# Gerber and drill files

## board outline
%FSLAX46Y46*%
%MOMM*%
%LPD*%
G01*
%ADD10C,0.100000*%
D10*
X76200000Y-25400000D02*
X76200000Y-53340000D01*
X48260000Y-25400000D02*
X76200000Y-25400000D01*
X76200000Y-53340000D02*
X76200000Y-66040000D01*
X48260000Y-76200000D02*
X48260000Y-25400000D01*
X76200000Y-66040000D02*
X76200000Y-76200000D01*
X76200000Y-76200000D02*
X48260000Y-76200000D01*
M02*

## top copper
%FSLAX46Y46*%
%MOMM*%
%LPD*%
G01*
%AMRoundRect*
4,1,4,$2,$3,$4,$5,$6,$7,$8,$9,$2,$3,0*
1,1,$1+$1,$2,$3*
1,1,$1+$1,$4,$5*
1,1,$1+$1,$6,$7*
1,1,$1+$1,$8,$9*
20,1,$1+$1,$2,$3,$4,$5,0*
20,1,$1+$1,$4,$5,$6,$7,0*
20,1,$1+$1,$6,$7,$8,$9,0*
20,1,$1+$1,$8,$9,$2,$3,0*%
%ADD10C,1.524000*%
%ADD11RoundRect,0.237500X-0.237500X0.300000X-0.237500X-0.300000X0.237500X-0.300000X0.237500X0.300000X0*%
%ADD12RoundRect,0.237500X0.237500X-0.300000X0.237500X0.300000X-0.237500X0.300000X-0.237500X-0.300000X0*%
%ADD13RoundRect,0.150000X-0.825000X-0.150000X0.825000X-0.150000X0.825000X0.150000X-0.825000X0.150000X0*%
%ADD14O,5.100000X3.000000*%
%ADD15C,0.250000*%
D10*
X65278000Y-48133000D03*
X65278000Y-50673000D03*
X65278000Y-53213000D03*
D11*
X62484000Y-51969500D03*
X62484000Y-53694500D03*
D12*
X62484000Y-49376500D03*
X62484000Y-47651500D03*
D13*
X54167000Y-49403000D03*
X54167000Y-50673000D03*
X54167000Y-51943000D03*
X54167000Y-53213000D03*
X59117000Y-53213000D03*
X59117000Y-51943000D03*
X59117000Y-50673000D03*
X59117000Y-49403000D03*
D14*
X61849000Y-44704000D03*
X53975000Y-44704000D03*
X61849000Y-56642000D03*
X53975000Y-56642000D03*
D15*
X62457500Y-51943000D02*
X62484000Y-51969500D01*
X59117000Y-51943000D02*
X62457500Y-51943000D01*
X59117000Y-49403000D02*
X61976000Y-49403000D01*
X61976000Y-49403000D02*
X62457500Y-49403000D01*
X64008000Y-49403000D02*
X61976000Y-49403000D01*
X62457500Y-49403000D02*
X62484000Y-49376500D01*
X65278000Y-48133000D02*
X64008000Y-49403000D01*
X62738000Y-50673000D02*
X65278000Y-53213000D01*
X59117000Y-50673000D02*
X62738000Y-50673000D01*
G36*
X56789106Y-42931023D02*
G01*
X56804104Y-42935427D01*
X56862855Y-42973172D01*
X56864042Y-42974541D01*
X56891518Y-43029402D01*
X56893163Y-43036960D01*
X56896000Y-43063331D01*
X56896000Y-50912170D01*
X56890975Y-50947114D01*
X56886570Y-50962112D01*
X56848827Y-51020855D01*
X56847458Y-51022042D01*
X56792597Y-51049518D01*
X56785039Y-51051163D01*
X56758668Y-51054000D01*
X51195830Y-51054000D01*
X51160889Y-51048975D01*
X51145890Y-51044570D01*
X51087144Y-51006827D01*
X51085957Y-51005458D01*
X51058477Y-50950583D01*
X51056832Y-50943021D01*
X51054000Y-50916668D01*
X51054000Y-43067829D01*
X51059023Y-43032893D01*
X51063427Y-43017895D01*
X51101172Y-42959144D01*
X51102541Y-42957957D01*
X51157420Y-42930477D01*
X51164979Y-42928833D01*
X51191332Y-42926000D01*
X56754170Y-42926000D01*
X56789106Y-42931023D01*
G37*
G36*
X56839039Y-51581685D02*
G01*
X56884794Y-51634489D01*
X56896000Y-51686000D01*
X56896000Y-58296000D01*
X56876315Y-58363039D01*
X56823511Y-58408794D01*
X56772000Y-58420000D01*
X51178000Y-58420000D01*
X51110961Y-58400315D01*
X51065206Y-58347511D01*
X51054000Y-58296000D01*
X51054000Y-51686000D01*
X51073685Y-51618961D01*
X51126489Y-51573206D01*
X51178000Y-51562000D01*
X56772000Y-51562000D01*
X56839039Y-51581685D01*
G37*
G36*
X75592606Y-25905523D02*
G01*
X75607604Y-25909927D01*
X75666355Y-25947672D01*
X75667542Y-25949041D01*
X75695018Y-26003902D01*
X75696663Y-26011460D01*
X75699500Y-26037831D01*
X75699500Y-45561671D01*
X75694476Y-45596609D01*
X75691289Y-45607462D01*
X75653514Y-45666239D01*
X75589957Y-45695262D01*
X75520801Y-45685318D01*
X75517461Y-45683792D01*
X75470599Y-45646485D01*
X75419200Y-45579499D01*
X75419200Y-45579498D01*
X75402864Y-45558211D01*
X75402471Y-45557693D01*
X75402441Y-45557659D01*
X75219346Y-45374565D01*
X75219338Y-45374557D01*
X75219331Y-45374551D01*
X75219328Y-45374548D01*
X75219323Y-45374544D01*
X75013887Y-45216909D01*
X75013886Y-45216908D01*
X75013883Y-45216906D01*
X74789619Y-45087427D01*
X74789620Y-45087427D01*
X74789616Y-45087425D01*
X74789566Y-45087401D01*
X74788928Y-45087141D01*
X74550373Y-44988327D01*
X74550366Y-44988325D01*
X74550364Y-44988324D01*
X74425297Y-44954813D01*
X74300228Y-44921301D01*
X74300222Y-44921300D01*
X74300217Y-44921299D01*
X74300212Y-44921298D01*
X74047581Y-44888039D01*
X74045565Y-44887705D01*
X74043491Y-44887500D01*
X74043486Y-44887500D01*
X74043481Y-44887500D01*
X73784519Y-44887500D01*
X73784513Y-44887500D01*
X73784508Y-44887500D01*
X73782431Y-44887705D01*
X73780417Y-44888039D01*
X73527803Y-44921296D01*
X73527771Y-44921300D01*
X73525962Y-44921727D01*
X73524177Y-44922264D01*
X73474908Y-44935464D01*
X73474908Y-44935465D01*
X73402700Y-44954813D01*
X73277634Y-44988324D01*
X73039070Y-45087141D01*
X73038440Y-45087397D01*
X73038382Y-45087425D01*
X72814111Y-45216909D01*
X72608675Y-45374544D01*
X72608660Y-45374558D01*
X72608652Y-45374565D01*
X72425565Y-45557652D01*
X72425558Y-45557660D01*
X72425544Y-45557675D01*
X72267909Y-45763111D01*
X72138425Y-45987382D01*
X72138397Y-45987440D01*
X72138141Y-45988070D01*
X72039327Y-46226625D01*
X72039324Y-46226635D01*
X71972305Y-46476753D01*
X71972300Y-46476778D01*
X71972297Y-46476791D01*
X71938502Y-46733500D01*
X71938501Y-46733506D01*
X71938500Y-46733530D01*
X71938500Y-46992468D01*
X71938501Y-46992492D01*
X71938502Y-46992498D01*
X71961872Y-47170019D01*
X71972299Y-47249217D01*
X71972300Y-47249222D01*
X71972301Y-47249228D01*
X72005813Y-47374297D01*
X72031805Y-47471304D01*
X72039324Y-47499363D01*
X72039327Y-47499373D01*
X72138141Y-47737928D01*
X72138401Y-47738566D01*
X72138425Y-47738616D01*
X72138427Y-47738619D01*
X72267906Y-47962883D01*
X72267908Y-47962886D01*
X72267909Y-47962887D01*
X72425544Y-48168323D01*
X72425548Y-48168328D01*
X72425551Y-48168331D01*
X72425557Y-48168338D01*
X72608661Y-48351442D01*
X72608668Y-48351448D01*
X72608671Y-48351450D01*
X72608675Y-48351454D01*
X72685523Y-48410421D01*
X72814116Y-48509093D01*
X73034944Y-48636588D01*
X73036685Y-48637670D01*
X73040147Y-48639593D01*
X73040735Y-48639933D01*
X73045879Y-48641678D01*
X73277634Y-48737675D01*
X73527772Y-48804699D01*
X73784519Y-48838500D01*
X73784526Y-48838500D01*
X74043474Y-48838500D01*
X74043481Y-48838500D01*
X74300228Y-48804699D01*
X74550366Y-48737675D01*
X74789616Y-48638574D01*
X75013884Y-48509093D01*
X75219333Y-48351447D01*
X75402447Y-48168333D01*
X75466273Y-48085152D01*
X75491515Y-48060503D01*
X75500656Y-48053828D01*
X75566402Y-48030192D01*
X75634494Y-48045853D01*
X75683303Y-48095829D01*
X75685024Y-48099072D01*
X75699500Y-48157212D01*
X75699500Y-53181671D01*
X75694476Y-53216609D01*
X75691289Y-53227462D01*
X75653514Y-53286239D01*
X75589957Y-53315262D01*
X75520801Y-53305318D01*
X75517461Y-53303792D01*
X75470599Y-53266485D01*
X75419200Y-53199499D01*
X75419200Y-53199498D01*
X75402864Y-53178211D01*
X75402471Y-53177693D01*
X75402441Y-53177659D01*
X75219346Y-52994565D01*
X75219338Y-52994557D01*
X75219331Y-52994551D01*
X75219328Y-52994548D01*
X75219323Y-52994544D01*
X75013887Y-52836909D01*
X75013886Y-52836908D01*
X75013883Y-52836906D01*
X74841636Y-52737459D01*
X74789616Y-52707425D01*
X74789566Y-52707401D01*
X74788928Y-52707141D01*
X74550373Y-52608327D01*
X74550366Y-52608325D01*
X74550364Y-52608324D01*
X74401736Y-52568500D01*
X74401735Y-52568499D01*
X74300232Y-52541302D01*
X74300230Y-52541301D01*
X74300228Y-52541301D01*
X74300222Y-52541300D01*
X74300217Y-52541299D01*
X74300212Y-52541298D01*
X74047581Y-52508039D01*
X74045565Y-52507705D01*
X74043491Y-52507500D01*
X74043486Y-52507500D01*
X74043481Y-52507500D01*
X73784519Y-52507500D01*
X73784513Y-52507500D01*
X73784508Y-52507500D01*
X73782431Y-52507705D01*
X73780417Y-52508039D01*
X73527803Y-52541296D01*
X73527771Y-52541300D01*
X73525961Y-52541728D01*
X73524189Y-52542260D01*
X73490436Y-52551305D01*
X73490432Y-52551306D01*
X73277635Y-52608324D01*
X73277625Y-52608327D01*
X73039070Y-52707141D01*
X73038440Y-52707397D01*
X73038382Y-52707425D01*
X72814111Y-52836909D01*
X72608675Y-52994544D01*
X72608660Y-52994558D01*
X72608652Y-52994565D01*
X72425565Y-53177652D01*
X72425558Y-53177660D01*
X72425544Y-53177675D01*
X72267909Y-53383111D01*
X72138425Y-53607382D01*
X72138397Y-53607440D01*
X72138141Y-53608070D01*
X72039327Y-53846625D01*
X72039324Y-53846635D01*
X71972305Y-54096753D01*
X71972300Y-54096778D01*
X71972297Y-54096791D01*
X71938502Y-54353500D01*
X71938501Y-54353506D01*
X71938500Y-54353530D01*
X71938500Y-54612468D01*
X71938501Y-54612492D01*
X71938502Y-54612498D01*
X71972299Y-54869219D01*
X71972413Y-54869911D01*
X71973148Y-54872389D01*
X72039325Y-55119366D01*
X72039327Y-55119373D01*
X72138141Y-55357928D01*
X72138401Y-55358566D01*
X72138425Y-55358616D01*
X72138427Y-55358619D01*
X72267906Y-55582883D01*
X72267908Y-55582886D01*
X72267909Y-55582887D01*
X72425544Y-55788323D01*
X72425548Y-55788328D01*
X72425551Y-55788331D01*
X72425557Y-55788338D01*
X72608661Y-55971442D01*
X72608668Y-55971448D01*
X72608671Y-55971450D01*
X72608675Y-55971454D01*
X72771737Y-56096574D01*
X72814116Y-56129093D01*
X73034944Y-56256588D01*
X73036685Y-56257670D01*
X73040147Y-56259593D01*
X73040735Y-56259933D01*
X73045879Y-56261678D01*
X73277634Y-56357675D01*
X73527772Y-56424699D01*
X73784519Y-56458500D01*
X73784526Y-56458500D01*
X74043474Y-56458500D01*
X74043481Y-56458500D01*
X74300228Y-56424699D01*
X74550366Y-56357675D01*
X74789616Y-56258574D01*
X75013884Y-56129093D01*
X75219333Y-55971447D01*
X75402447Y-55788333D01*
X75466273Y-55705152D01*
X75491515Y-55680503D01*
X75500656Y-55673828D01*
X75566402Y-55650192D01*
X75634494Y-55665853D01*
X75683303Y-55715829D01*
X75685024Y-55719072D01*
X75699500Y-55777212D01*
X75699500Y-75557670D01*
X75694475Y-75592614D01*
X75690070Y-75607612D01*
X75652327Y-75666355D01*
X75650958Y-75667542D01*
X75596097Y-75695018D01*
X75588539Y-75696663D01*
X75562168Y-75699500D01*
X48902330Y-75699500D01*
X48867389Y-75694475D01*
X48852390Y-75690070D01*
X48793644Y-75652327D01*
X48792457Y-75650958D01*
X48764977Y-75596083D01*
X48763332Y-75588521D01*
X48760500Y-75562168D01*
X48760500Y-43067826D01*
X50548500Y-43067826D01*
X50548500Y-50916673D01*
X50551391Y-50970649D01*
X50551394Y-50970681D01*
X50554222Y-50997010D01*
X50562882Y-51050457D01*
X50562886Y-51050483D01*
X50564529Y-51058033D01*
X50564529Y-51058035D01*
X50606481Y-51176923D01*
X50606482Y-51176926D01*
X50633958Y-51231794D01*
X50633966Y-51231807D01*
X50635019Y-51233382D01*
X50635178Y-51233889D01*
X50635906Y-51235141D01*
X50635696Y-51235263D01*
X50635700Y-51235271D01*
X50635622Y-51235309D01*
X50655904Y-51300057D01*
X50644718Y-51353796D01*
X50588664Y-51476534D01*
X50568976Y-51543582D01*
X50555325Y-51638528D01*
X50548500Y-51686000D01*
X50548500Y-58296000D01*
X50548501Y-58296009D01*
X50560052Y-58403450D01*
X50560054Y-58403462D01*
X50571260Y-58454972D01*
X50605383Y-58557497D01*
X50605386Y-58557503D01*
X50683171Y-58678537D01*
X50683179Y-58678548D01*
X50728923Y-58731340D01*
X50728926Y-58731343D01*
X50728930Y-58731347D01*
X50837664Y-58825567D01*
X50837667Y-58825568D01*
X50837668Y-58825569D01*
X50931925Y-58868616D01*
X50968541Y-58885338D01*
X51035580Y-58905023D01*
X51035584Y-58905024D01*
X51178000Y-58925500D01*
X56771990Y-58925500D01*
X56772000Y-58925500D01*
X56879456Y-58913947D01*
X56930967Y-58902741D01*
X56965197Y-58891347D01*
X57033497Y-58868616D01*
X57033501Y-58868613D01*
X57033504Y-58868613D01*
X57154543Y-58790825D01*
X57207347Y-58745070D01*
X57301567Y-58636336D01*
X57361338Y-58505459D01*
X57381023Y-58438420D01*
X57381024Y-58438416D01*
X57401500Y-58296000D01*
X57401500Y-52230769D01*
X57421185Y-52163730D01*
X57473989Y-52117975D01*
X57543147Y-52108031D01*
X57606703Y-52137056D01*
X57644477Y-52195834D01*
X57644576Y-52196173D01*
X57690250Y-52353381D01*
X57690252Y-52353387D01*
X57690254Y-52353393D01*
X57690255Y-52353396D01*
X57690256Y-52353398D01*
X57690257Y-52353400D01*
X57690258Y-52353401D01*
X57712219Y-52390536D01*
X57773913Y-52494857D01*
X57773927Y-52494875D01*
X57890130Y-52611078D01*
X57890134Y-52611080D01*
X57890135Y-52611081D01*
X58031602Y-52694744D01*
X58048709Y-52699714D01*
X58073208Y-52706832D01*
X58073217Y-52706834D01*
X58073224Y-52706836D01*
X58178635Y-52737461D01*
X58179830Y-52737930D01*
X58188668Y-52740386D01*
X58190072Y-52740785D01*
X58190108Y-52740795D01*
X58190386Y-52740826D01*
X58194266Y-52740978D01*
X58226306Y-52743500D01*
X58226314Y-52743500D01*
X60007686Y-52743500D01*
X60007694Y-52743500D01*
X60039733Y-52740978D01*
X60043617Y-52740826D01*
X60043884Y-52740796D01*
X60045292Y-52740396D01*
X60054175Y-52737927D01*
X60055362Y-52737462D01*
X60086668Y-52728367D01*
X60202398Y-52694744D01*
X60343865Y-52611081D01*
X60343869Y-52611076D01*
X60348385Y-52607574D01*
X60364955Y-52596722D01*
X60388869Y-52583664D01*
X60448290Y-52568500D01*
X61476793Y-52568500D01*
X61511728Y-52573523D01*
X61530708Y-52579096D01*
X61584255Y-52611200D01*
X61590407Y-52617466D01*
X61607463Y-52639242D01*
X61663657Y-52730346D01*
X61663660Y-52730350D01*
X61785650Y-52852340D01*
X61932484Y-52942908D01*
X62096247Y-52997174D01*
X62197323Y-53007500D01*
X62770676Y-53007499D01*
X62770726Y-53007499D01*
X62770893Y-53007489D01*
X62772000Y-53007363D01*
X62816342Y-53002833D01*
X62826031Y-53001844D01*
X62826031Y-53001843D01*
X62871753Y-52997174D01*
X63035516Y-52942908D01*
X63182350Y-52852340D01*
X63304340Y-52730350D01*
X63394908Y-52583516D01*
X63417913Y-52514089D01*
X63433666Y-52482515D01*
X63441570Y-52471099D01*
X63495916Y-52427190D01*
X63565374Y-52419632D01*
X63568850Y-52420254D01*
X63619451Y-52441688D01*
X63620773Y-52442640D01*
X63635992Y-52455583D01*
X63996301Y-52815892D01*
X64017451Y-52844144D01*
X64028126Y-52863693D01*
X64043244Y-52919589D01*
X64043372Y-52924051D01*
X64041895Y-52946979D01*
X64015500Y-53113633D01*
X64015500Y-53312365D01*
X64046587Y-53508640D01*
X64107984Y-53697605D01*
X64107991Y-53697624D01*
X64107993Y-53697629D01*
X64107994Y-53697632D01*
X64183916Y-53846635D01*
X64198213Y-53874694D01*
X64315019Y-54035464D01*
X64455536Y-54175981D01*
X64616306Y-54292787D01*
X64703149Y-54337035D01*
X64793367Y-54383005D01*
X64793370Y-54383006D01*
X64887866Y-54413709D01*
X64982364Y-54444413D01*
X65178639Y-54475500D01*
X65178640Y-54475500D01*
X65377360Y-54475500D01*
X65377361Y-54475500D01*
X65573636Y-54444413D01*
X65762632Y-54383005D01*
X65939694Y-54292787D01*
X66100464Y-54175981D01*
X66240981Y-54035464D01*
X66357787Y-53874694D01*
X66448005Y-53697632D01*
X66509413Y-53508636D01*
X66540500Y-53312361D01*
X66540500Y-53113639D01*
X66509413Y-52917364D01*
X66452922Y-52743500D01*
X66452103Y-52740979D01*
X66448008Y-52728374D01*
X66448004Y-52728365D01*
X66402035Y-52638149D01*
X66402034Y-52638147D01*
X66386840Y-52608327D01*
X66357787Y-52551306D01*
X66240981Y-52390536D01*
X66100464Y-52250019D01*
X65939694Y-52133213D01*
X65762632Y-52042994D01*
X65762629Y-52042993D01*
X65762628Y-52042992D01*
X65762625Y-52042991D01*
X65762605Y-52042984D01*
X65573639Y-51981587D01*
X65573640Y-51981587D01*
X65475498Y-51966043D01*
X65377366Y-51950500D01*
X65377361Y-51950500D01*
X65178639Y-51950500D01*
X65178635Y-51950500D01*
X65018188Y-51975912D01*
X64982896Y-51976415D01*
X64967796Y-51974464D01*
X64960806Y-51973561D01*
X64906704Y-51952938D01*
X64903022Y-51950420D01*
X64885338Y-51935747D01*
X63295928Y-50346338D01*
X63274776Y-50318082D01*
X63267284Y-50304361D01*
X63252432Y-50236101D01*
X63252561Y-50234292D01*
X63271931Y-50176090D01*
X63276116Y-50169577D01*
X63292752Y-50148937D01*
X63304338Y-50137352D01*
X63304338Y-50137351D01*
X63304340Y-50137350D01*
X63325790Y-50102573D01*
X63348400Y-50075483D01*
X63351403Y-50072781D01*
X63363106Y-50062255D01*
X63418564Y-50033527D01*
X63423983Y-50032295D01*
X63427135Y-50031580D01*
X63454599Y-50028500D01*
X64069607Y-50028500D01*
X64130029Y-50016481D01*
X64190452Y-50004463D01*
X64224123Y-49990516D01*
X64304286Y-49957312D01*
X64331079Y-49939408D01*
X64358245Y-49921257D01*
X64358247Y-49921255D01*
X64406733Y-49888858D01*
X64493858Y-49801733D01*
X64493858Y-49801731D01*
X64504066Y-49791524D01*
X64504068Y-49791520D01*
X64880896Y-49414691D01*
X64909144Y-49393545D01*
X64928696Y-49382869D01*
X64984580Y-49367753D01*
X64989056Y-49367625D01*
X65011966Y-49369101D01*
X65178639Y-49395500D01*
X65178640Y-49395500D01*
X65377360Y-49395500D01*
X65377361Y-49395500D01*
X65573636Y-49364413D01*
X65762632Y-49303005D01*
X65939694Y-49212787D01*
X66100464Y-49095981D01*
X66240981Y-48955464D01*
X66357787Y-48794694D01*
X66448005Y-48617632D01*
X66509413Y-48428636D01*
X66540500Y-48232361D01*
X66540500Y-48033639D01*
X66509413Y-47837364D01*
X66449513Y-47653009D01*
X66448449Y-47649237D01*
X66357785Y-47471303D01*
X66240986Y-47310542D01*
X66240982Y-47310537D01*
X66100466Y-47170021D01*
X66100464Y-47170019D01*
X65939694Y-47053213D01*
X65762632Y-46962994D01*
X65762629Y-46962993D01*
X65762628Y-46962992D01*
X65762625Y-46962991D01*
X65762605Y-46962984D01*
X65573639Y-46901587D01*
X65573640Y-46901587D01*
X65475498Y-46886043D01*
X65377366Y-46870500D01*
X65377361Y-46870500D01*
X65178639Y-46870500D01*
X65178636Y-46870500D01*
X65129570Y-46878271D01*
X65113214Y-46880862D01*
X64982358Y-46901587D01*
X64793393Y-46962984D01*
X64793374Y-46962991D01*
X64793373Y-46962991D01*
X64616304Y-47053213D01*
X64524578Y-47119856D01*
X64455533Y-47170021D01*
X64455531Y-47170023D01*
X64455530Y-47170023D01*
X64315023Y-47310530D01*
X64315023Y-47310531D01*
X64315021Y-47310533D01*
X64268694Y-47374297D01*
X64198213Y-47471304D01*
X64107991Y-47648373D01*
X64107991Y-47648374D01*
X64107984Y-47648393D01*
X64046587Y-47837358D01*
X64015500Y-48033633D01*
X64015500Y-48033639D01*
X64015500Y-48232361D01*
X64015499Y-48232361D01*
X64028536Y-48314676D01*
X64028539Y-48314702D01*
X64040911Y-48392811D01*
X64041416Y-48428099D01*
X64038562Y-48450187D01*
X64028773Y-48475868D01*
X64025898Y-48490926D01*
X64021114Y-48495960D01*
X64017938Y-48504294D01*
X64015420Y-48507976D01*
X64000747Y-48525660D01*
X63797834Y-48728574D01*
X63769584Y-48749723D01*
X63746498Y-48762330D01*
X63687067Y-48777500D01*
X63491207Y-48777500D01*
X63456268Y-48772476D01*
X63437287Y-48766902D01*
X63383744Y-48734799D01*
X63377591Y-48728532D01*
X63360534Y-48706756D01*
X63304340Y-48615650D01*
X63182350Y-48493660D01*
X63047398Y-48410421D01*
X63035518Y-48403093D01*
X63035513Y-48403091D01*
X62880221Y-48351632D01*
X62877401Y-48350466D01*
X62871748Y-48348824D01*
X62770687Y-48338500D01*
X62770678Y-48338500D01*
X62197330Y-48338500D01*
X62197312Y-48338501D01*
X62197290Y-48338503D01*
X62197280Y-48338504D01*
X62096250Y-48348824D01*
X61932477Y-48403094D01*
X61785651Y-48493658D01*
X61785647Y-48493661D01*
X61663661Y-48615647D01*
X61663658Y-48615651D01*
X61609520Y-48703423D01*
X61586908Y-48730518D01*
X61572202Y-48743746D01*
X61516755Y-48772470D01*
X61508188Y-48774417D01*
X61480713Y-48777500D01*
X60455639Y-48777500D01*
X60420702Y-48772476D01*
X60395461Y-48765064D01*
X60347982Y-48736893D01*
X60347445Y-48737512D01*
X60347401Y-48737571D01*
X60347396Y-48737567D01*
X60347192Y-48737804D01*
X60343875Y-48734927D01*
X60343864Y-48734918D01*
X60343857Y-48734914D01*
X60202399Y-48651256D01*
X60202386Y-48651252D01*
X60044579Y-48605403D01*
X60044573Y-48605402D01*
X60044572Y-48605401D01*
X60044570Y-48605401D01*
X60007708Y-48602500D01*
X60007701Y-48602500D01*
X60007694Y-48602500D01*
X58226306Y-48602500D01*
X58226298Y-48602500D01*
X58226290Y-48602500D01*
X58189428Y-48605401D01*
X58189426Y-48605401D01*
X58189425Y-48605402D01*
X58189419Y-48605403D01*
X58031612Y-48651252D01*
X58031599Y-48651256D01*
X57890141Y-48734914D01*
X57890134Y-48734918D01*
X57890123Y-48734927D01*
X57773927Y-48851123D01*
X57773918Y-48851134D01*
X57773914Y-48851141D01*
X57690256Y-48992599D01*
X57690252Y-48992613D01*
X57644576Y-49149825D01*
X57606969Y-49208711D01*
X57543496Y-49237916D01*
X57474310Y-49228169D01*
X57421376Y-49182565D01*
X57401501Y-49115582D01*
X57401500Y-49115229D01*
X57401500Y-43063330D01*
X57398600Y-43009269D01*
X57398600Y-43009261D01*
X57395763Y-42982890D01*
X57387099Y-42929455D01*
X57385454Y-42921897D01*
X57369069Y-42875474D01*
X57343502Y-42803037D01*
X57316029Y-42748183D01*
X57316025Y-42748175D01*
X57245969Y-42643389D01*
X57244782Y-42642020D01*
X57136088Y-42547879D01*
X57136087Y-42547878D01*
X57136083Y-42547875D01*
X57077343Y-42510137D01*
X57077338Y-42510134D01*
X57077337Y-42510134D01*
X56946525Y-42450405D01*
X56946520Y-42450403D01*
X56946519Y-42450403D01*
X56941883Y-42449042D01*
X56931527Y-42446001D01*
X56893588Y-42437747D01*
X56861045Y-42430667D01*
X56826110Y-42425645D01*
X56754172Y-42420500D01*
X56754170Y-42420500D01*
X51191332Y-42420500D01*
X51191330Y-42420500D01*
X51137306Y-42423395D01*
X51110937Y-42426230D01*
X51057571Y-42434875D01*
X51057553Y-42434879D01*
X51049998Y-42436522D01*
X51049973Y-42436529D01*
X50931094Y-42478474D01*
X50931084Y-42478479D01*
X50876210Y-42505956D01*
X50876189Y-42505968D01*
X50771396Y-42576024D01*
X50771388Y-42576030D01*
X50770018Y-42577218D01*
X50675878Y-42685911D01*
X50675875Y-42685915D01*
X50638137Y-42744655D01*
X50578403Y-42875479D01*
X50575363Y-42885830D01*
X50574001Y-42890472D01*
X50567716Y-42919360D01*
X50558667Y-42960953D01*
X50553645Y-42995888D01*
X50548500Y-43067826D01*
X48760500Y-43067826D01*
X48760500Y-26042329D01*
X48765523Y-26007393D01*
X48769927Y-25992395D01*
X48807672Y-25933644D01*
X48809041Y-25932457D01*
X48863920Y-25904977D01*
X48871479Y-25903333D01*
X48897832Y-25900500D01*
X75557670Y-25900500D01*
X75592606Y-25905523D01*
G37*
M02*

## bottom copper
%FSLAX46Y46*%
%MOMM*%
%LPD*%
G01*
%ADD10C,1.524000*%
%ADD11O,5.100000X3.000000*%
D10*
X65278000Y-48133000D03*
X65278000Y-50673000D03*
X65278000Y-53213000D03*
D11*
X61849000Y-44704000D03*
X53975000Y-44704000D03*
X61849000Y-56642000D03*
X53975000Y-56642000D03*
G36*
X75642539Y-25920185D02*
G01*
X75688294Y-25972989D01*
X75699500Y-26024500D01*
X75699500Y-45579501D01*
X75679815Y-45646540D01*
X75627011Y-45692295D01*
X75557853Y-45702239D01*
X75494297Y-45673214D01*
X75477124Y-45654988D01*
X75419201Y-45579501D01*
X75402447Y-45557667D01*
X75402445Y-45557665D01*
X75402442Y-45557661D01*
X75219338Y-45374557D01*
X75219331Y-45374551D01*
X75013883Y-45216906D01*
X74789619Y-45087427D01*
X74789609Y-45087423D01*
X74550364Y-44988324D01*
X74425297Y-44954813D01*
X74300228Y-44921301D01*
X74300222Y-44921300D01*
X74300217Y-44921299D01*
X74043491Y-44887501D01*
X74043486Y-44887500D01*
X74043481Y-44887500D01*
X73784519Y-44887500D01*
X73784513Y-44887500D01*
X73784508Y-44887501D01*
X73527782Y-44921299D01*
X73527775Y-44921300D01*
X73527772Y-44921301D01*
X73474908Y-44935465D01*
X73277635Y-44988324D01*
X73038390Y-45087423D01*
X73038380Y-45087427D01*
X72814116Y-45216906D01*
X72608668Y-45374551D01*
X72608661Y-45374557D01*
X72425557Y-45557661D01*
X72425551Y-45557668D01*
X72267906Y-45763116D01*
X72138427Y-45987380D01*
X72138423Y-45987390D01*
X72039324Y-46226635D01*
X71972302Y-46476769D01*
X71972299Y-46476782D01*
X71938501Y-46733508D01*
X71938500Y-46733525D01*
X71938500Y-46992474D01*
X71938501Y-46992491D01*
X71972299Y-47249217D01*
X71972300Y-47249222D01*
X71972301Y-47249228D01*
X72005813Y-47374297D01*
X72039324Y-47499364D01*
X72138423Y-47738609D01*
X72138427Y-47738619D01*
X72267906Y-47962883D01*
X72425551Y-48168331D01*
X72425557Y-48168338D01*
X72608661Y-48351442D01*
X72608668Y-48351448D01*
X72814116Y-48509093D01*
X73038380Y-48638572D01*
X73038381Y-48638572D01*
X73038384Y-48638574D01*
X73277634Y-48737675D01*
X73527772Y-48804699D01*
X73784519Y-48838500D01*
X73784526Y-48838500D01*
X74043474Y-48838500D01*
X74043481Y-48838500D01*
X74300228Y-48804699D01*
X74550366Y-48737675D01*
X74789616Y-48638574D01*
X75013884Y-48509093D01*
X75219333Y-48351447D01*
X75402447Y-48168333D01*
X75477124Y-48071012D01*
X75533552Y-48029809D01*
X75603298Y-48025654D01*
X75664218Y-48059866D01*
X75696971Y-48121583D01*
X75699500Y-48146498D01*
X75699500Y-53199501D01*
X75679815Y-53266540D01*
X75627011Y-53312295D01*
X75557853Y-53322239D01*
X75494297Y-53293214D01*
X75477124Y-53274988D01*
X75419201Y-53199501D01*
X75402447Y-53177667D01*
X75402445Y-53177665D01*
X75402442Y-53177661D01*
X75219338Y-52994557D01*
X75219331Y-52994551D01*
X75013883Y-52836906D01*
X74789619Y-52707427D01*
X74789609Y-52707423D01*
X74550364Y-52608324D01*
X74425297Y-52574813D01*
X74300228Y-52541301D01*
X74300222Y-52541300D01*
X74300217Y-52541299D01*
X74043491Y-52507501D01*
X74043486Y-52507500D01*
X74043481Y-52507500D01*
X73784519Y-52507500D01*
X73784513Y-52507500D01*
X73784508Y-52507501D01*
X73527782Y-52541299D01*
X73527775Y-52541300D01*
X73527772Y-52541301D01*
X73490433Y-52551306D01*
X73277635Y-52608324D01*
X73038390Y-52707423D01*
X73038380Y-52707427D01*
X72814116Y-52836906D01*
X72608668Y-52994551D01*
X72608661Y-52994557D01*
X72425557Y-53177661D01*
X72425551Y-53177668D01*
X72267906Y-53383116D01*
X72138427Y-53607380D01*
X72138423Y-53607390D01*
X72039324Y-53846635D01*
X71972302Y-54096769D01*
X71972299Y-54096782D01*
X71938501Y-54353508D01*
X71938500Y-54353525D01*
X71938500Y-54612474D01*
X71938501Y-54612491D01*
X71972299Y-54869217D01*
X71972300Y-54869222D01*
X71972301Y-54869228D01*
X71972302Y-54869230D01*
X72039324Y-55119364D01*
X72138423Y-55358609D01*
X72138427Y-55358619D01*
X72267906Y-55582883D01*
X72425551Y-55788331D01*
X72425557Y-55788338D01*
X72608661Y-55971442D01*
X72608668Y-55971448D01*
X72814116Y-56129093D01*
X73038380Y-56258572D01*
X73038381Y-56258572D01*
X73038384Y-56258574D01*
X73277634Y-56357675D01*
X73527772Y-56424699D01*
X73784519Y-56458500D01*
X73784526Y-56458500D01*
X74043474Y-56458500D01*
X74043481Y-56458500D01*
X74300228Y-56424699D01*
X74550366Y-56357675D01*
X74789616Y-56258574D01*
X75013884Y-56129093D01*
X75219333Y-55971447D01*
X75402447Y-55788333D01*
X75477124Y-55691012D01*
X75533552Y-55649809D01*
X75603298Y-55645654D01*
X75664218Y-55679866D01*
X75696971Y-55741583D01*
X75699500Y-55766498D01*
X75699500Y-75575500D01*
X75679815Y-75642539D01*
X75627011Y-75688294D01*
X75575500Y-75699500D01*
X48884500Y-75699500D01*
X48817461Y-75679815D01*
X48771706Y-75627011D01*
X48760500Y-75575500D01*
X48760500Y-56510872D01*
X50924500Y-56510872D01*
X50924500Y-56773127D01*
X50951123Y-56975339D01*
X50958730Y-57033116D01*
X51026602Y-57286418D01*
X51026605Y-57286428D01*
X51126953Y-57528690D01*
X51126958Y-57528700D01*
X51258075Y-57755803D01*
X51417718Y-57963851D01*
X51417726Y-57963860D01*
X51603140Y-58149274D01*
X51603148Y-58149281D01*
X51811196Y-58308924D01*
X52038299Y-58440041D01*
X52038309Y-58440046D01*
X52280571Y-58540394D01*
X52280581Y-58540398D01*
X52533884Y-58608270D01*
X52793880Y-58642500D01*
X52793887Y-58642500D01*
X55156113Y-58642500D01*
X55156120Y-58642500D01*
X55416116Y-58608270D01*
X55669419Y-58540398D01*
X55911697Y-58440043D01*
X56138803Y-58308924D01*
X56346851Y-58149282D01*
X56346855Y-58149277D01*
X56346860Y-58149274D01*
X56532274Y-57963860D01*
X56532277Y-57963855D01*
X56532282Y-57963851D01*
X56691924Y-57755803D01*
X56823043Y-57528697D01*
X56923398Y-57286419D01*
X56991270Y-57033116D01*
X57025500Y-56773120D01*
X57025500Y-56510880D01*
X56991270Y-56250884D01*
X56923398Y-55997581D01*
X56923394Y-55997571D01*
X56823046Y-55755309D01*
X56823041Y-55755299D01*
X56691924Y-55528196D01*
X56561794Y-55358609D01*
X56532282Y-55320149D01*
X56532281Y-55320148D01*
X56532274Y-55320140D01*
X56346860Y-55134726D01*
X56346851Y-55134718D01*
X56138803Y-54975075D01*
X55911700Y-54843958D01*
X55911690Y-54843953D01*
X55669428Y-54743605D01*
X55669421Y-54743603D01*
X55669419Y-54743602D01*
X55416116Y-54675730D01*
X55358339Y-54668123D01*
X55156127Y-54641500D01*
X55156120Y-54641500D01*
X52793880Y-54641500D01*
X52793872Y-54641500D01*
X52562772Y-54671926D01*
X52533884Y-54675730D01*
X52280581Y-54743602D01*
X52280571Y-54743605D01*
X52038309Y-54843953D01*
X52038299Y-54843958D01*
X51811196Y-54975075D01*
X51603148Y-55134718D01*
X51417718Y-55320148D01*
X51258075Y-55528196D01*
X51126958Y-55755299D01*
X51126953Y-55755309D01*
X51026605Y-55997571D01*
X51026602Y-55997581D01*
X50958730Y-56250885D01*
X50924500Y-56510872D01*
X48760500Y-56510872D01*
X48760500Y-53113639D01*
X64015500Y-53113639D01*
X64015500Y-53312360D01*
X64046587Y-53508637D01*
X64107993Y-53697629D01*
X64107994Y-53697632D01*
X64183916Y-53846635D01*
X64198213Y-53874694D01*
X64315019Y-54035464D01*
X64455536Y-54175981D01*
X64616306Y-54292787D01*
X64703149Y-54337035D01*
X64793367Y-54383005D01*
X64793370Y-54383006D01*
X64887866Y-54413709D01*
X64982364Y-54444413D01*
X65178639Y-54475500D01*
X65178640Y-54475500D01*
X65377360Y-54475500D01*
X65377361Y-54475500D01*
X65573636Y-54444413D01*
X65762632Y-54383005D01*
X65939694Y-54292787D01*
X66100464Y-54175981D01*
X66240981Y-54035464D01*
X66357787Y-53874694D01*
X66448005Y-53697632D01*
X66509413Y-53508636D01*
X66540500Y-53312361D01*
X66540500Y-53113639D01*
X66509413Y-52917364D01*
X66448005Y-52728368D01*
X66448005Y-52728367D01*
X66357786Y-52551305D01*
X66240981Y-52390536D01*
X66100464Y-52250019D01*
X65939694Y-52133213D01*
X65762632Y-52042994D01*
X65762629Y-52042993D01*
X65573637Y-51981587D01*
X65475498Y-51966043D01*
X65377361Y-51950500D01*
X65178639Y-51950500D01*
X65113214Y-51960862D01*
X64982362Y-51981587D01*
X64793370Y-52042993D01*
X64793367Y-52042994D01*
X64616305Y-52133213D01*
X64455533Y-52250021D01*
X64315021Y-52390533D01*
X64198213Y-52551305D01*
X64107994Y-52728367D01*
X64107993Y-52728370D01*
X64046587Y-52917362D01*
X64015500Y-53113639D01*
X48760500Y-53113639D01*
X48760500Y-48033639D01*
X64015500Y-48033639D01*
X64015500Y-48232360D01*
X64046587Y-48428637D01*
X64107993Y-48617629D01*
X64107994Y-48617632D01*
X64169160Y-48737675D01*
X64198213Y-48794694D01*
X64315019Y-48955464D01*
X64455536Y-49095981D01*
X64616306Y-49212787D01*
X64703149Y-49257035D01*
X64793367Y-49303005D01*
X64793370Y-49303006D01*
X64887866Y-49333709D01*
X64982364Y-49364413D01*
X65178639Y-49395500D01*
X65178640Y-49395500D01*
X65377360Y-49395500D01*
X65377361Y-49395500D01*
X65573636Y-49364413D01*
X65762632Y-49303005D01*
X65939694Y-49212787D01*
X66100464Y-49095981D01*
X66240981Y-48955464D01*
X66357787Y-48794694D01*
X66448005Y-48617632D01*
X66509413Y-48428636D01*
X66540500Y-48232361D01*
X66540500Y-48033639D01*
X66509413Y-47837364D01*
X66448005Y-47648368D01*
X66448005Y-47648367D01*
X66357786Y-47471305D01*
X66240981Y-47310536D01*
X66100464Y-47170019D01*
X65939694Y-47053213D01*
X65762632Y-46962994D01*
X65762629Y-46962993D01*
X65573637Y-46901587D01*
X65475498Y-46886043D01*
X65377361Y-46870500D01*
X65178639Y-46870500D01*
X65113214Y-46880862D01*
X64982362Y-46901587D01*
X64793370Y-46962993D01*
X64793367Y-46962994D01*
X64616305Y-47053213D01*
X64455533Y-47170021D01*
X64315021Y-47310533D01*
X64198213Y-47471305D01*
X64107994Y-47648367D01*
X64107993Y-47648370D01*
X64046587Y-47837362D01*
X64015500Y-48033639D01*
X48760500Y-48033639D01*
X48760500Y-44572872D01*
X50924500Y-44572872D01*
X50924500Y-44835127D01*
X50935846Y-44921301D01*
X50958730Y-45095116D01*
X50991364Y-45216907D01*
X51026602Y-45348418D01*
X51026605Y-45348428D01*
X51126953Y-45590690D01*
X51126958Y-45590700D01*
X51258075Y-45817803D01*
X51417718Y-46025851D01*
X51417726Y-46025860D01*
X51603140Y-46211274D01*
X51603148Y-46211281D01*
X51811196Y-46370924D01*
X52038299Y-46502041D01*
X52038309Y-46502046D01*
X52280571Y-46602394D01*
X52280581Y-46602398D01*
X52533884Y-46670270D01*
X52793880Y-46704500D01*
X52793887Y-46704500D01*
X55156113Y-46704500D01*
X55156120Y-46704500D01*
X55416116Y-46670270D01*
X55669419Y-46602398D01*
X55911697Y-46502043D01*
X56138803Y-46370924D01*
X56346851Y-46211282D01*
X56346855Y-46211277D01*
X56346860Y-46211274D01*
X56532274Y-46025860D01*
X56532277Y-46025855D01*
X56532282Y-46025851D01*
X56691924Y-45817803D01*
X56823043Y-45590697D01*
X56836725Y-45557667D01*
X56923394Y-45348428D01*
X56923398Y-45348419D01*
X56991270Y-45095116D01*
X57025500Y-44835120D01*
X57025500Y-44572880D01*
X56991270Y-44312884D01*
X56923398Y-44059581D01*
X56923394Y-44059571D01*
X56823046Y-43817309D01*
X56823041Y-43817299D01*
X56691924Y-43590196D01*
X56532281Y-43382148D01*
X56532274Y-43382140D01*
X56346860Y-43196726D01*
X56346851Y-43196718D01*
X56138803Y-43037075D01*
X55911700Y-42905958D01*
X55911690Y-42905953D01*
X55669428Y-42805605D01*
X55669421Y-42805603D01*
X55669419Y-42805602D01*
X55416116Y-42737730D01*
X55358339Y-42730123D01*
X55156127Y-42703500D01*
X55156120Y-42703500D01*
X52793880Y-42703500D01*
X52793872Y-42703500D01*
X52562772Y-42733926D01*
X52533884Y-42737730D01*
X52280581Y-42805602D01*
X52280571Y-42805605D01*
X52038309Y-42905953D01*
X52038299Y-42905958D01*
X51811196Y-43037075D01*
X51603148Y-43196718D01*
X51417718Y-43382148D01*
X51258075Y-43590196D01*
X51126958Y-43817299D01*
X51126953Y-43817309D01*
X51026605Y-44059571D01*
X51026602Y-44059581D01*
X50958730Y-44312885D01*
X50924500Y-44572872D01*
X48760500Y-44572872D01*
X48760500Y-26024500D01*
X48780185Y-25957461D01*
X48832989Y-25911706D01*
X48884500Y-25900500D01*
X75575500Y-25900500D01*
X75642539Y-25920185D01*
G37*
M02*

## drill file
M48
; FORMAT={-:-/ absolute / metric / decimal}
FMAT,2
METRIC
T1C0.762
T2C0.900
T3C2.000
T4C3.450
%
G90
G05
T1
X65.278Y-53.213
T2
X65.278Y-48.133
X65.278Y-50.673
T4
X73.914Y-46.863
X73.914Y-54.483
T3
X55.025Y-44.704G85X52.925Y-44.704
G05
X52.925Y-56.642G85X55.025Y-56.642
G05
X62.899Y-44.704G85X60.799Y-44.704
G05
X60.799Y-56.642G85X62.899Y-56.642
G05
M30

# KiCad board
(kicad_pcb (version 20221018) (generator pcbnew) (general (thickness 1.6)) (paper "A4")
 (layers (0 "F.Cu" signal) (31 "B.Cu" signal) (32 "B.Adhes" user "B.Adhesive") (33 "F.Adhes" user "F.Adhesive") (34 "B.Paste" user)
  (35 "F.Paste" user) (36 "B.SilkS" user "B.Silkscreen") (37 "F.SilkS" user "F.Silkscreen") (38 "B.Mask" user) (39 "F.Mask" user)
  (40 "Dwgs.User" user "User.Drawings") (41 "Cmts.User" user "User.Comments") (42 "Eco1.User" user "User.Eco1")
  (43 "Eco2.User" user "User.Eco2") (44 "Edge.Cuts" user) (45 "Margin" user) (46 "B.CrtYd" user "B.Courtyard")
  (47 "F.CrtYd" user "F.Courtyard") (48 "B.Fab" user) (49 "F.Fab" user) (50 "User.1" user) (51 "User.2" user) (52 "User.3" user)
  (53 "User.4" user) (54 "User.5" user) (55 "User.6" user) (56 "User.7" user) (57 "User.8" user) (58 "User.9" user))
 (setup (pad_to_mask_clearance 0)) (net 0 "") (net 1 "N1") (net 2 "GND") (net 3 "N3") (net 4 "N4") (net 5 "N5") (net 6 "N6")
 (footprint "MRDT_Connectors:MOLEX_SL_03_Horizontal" (layer "F.Cu") (at 65.278 48.133 -90)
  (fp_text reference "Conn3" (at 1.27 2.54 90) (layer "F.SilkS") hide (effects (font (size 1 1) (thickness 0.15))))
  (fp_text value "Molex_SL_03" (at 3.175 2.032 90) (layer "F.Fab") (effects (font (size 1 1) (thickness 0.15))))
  (pad "" np_thru_hole circle (at -1.27 -8.636 270) (size 3.45 3.45) (drill 3.45) (layers "*.Cu" "*.Mask"))
  (pad "" np_thru_hole circle (at 6.35 -8.636 270) (size 3.45 3.45) (drill 3.45) (layers "*.Cu" "*.Mask"))
  (pad "1" thru_hole circle (at 0 0 270) (size 1.524 1.524) (drill 0.9) (layers "*.Cu" "*.Mask") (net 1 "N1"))
  (pad "2" thru_hole circle (at 2.54 0 270) (size 1.524 1.524) (drill 0.9) (layers "*.Cu" "*.Mask") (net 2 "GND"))
  (pad "3" thru_hole circle (at 5.08 0 270) (size 1.524 1.524) (drill 0.762) (layers "*.Cu" "*.Mask") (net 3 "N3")))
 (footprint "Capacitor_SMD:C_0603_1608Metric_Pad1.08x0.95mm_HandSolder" (layer "F.Cu") (at 62.484 52.832 -90)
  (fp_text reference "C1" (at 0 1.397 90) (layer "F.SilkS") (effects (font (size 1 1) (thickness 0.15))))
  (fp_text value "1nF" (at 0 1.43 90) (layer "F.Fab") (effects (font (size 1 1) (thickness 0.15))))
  (pad "1" smd roundrect (at -0.8625 0 270) (size 1.075 0.95) (layers "F.Cu" "F.Paste" "F.Mask") (roundrect_rratio 0.25) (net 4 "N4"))
  (pad "2" smd roundrect (at 0.8625 0 270) (size 1.075 0.95) (layers "F.Cu" "F.Paste" "F.Mask") (roundrect_rratio 0.25) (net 2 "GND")))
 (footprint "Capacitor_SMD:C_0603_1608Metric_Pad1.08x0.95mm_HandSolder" (layer "F.Cu") (at 62.484 48.514 90)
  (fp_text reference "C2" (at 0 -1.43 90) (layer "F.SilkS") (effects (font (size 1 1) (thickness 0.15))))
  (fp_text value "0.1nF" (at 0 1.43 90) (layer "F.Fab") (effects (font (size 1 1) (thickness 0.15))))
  (pad "1" smd roundrect (at -0.8625 0 90) (size 1.075 0.95) (layers "F.Cu" "F.Paste" "F.Mask") (roundrect_rratio 0.25) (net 1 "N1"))
  (pad "2" smd roundrect (at 0.8625 0 90) (size 1.075 0.95) (layers "F.Cu" "F.Paste" "F.Mask") (roundrect_rratio 0.25) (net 2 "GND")))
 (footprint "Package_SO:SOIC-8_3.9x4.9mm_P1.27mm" (layer "F.Cu") (at 56.642 51.308)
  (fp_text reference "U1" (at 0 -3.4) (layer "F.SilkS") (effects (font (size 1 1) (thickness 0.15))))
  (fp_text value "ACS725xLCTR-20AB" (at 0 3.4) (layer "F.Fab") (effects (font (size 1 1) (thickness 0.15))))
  (pad "1" smd roundrect (at -2.475 -1.905) (size 1.95 0.6) (layers "F.Cu" "F.Paste" "F.Mask") (roundrect_rratio 0.25) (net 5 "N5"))
  (pad "2" smd roundrect (at -2.475 -0.635) (size 1.95 0.6) (layers "F.Cu" "F.Paste" "F.Mask") (roundrect_rratio 0.25) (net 5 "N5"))
  (pad "3" smd roundrect (at -2.475 0.635) (size 1.95 0.6) (layers "F.Cu" "F.Paste" "F.Mask") (roundrect_rratio 0.25) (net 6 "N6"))
  (pad "4" smd roundrect (at -2.475 1.905) (size 1.95 0.6) (layers "F.Cu" "F.Paste" "F.Mask") (roundrect_rratio 0.25) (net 6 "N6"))
  (pad "5" smd roundrect (at 2.475 1.905) (size 1.95 0.6) (layers "F.Cu" "F.Paste" "F.Mask") (roundrect_rratio 0.25) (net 2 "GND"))
  (pad "6" smd roundrect (at 2.475 0.635) (size 1.95 0.6) (layers "F.Cu" "F.Paste" "F.Mask") (roundrect_rratio 0.25) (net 4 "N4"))
  (pad "7" smd roundrect (at 2.475 -0.635) (size 1.95 0.6) (layers "F.Cu" "F.Paste" "F.Mask") (roundrect_rratio 0.25) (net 3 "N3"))
  (pad "8" smd roundrect (at 2.475 -1.905) (size 1.95 0.6) (layers "F.Cu" "F.Paste" "F.Mask") (roundrect_rratio 0.25) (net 1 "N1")))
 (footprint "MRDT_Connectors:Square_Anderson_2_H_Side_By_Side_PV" (layer "F.Cu") (at 62.149 44.8286 -90)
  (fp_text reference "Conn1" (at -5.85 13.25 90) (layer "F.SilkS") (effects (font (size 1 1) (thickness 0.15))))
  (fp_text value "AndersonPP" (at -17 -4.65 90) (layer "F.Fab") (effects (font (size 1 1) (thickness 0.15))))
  (pad "1" thru_hole oval (at -0.1246 0.3 270) (size 3 5.1) (drill oval 2 4.1) (layers "*.Cu" "*.Mask") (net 2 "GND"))
  (pad "4" thru_hole oval (at -0.1246 8.174 270) (size 3 5.1) (drill oval 2 4.1) (layers "*.Cu" "*.Mask") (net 5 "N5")))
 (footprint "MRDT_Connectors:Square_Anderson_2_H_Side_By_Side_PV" (layer "B.Cu") (at 62.149 56.5174 90)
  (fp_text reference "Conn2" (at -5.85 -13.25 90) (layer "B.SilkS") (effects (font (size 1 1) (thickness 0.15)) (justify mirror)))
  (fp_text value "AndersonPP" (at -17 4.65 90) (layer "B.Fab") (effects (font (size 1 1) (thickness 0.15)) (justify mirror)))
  (pad "1" thru_hole oval (at -0.1246 -0.3 90) (size 3 5.1) (drill oval 2 4.1) (layers "*.Cu" "*.Mask") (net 2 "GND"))
  (pad "4" thru_hole oval (at -0.1246 -8.174 90) (size 3 5.1) (drill oval 2 4.1) (layers "*.Cu" "*.Mask") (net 6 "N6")))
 (gr_line (start 76.2 25.4) (end 76.2 53.34) (stroke (width 0.1) (type default)) (layer "Edge.Cuts"))
 (gr_line (start 48.26 25.4) (end 76.2 25.4) (stroke (width 0.1) (type default)) (layer "Edge.Cuts"))
 (gr_line (start 76.2 53.34) (end 76.2 66.04) (stroke (width 0.1) (type default)) (layer "Edge.Cuts"))
 (gr_line (start 48.26 76.2) (end 48.26 25.4) (stroke (width 0.1) (type default)) (layer "Edge.Cuts"))
 (gr_line (start 76.2 66.04) (end 76.2 76.2) (stroke (width 0.1) (type default)) (layer "Edge.Cuts"))
 (gr_line (start 76.2 76.2) (end 48.26 76.2) (stroke (width 0.1) (type default)) (layer "Edge.Cuts"))
 (segment (start 62.4575 51.943) (end 62.484 51.9695) (width 0.25) (layer "F.Cu") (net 4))
 (segment (start 59.117 51.943) (end 62.4575 51.943) (width 0.25) (layer "F.Cu") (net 4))
 (segment (start 59.117 49.403) (end 61.976 49.403) (width 0.25) (layer "F.Cu") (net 1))
 (segment (start 61.976 49.403) (end 62.4575 49.403) (width 0.25) (layer "F.Cu") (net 1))
 (segment (start 64.008 49.403) (end 61.976 49.403) (width 0.25) (layer "F.Cu") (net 1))
 (segment (start 62.4575 49.403) (end 62.484 49.3765) (width 0.25) (layer "F.Cu") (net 1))
 (segment (start 65.278 48.133) (end 64.008 49.403) (width 0.25) (layer "F.Cu") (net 1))
 (segment (start 62.738 50.673) (end 65.278 53.213) (width 0.25) (layer "F.Cu") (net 3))
 (segment (start 59.117 50.673) (end 62.738 50.673) (width 0.25) (layer "F.Cu") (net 3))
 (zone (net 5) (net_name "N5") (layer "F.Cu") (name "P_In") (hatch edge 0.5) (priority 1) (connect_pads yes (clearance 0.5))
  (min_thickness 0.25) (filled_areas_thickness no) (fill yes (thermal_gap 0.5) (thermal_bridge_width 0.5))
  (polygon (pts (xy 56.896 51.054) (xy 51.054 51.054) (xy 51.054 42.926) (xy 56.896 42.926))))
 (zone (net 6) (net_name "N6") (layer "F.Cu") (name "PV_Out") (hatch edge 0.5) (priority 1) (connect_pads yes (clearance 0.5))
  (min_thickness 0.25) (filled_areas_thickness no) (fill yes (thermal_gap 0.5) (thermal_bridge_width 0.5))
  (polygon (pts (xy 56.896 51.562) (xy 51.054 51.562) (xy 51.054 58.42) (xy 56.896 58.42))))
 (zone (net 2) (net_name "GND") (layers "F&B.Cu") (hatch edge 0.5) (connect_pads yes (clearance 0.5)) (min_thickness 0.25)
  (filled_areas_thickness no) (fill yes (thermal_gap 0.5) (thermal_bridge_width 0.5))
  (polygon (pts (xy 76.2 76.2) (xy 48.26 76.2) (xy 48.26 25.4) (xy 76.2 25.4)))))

